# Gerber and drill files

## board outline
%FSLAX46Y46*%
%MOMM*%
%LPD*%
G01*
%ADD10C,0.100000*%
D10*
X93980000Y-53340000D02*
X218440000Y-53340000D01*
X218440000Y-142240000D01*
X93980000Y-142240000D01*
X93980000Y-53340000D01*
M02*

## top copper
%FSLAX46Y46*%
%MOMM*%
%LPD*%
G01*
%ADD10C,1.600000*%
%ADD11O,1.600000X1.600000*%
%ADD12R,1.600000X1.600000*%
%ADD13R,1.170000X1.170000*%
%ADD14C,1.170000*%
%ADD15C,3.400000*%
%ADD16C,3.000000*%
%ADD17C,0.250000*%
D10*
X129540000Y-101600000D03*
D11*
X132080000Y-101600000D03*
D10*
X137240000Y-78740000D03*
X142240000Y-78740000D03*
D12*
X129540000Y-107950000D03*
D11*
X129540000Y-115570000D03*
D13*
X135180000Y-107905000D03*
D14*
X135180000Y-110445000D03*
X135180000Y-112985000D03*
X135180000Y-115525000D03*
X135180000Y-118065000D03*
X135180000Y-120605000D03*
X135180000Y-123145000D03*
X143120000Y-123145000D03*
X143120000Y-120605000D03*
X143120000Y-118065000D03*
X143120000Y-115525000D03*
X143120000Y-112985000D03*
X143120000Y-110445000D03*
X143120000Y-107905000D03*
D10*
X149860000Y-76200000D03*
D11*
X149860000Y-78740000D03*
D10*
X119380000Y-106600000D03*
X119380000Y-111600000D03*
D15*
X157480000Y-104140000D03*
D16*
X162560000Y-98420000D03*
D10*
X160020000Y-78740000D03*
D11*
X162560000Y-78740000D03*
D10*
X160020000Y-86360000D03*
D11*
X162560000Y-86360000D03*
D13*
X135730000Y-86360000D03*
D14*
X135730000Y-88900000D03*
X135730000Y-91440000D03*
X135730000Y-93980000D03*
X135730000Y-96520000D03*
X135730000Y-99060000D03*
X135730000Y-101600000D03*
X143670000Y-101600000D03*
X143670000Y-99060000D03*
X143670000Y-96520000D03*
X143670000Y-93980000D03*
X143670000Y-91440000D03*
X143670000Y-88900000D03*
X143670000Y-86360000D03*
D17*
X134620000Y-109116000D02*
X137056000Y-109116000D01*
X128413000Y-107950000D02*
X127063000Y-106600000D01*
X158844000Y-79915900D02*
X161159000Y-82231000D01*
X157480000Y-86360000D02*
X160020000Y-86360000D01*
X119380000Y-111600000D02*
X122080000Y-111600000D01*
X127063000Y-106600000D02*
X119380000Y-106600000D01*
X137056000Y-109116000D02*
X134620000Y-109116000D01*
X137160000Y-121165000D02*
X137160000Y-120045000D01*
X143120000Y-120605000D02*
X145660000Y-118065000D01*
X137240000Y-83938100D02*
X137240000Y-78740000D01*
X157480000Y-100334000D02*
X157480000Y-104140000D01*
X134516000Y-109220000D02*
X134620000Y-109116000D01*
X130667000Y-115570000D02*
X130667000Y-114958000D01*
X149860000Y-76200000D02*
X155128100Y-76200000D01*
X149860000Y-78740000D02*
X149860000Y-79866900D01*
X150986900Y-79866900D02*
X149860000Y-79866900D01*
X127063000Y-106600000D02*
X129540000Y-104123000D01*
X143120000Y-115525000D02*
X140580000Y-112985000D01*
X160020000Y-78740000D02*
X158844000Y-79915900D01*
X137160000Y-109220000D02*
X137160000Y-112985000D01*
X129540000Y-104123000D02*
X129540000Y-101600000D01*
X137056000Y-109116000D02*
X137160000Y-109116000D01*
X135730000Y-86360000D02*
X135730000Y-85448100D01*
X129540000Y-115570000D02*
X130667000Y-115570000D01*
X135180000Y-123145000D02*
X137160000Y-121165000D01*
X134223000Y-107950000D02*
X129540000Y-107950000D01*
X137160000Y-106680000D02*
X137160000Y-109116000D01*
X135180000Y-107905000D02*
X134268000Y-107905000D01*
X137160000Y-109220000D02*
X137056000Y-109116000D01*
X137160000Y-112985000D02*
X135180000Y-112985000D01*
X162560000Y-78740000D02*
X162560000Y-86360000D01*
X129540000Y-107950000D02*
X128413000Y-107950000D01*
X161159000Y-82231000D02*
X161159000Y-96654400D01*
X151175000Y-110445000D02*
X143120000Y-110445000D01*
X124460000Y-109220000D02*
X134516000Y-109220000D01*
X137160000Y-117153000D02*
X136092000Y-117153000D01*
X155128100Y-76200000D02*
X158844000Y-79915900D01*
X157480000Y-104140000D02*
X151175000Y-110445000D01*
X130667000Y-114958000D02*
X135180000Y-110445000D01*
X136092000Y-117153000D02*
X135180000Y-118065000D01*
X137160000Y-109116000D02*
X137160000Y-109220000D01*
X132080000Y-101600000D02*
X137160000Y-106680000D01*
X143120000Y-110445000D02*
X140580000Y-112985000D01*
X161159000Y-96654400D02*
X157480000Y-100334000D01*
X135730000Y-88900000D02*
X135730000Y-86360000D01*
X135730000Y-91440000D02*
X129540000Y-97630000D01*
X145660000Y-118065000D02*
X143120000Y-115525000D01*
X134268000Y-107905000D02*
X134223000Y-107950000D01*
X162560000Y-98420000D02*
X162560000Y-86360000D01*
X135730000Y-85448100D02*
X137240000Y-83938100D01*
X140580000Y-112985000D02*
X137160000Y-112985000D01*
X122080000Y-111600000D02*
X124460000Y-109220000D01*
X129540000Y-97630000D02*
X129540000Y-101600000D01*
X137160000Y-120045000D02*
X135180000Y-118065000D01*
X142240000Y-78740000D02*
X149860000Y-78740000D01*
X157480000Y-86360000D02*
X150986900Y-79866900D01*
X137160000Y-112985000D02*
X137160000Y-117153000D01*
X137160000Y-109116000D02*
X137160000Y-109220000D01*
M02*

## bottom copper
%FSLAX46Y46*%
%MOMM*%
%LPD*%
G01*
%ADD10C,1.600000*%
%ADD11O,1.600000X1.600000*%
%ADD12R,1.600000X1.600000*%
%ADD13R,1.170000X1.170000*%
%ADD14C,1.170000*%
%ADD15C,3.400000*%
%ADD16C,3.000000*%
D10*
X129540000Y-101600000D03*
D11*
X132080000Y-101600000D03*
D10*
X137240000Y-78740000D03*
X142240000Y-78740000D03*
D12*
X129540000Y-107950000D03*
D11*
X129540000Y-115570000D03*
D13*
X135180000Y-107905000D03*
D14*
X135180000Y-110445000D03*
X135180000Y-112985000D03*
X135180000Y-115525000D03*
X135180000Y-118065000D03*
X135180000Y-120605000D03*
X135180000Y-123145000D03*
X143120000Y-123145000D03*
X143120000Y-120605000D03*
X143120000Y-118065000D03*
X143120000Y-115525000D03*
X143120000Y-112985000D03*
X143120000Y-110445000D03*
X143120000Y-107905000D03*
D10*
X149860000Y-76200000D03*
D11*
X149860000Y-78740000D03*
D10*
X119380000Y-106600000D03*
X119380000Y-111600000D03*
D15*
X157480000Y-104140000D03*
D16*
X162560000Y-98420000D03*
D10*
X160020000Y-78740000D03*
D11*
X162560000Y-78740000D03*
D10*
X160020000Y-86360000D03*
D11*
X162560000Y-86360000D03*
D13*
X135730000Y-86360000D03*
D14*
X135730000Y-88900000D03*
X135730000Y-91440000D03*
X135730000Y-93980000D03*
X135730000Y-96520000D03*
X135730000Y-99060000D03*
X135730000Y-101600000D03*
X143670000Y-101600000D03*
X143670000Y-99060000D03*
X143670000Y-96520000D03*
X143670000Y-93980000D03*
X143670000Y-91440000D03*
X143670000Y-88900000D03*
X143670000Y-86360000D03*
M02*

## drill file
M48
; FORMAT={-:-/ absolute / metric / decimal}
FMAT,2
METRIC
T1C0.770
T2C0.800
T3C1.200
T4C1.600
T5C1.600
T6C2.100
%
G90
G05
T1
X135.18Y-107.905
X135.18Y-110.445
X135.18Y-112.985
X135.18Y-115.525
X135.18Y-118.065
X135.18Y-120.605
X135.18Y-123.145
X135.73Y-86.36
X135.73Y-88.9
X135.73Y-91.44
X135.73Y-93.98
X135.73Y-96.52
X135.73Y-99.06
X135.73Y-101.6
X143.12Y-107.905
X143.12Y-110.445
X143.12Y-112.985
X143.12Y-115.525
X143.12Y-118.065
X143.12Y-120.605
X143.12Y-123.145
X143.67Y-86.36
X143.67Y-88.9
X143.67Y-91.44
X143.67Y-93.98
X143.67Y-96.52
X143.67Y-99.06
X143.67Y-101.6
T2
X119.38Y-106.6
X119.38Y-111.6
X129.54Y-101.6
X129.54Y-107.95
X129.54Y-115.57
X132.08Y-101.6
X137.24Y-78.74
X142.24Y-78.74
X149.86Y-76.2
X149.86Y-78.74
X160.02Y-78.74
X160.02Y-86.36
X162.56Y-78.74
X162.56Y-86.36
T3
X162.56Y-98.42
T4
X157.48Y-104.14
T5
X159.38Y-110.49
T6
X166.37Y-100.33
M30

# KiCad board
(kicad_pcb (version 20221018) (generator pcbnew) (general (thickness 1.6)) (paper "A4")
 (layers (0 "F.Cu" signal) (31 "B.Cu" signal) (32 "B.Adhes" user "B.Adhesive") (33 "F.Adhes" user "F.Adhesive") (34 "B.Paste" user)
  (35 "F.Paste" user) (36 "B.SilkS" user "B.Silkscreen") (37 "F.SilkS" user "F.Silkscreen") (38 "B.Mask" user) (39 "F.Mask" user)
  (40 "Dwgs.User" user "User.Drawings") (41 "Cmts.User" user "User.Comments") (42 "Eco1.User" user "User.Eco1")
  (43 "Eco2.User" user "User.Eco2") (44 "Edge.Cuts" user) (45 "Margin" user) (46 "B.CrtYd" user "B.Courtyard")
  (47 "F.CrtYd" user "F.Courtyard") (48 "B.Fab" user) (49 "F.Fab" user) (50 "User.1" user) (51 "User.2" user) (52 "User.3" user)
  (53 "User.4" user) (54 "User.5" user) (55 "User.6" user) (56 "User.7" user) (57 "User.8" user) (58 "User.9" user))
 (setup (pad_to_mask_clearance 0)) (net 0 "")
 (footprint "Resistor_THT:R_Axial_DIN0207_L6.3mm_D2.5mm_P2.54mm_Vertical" (layer "F.Cu") (at 129.54 101.6)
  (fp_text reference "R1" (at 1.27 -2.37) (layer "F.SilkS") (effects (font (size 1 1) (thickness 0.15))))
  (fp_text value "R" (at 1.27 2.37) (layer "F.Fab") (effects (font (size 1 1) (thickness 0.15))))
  (pad "1" thru_hole circle (at 0 0) (size 1.6 1.6) (drill 0.8) (layers "*.Cu" "*.Mask"))
  (pad "2" thru_hole oval (at 2.54 0) (size 1.6 1.6) (drill 0.8) (layers "*.Cu" "*.Mask")))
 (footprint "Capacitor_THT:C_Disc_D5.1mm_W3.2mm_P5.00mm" (layer "F.Cu") (at 137.24 78.74)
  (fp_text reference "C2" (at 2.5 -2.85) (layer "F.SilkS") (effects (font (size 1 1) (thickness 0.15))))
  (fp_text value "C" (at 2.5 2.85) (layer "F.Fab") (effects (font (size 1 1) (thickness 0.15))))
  (pad "1" thru_hole circle (at 0 0) (size 1.6 1.6) (drill 0.8) (layers "*.Cu" "*.Mask"))
  (pad "2" thru_hole circle (at 5 0) (size 1.6 1.6) (drill 0.8) (layers "*.Cu" "*.Mask")))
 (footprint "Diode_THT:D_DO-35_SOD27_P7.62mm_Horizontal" (layer "F.Cu") (at 129.54 107.95 -90)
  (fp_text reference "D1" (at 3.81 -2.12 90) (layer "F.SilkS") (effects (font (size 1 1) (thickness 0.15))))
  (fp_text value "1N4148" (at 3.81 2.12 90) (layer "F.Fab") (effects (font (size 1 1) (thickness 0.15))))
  (pad "1" thru_hole rect (at 0 0 270) (size 1.6 1.6) (drill 0.8) (layers "*.Cu" "*.Mask"))
  (pad "2" thru_hole oval (at 7.62 0 270) (size 1.6 1.6) (drill 0.8) (layers "*.Cu" "*.Mask")))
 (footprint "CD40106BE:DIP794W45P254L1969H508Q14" (layer "F.Cu") (at 139.15 115.525)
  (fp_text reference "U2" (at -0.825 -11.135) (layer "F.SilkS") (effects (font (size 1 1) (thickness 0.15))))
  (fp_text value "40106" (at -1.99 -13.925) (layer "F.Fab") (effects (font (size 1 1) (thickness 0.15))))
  (pad "1" thru_hole rect (at -3.97 -7.62) (size 1.17 1.17) (drill 0.77) (layers "*.Cu" "*.Mask") (solder_mask_margin 0.102))
  (pad "2" thru_hole circle (at -3.97 -5.08) (size 1.17 1.17) (drill 0.77) (layers "*.Cu" "*.Mask") (solder_mask_margin 0.102))
  (pad "3" thru_hole circle (at -3.97 -2.54) (size 1.17 1.17) (drill 0.77) (layers "*.Cu" "*.Mask") (solder_mask_margin 0.102))
  (pad "4" thru_hole circle (at -3.97 0) (size 1.17 1.17) (drill 0.77) (layers "*.Cu" "*.Mask") (solder_mask_margin 0.102))
  (pad "5" thru_hole circle (at -3.97 2.54) (size 1.17 1.17) (drill 0.77) (layers "*.Cu" "*.Mask") (solder_mask_margin 0.102))
  (pad "6" thru_hole circle (at -3.97 5.08) (size 1.17 1.17) (drill 0.77) (layers "*.Cu" "*.Mask") (solder_mask_margin 0.102))
  (pad "7" thru_hole circle (at -3.97 7.62) (size 1.17 1.17) (drill 0.77) (layers "*.Cu" "*.Mask") (solder_mask_margin 0.102))
  (pad "8" thru_hole circle (at 3.97 7.62) (size 1.17 1.17) (drill 0.77) (layers "*.Cu" "*.Mask") (solder_mask_margin 0.102))
  (pad "9" thru_hole circle (at 3.97 5.08) (size 1.17 1.17) (drill 0.77) (layers "*.Cu" "*.Mask") (solder_mask_margin 0.102))
  (pad "10" thru_hole circle (at 3.97 2.54) (size 1.17 1.17) (drill 0.77) (layers "*.Cu" "*.Mask") (solder_mask_margin 0.102))
  (pad "11" thru_hole circle (at 3.97 0) (size 1.17 1.17) (drill 0.77) (layers "*.Cu" "*.Mask") (solder_mask_margin 0.102))
  (pad "12" thru_hole circle (at 3.97 -2.54) (size 1.17 1.17) (drill 0.77) (layers "*.Cu" "*.Mask") (solder_mask_margin 0.102))
  (pad "13" thru_hole circle (at 3.97 -5.08) (size 1.17 1.17) (drill 0.77) (layers "*.Cu" "*.Mask") (solder_mask_margin 0.102))
  (pad "14" thru_hole circle (at 3.97 -7.62) (size 1.17 1.17) (drill 0.77) (layers "*.Cu" "*.Mask") (solder_mask_margin 0.102)))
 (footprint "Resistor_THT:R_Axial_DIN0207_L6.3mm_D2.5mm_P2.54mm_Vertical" (layer "F.Cu") (at 149.86 76.2 -90)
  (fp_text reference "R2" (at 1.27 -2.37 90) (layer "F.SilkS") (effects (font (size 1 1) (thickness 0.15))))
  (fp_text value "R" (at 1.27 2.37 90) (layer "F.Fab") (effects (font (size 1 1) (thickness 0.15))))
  (pad "1" thru_hole circle (at 0 0 270) (size 1.6 1.6) (drill 0.8) (layers "*.Cu" "*.Mask"))
  (pad "2" thru_hole oval (at 2.54 0 270) (size 1.6 1.6) (drill 0.8) (layers "*.Cu" "*.Mask")))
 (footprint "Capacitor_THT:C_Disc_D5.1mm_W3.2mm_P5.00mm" (layer "F.Cu") (at 119.38 106.6 -90)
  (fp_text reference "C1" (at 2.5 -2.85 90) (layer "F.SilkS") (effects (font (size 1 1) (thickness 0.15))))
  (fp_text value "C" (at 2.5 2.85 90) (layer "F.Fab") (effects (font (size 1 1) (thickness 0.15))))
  (pad "1" thru_hole circle (at 0 0 270) (size 1.6 1.6) (drill 0.8) (layers "*.Cu" "*.Mask"))
  (pad "2" thru_hole circle (at 5 0 270) (size 1.6 1.6) (drill 0.8) (layers "*.Cu" "*.Mask")))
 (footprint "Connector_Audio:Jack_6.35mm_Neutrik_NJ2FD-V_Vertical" (layer "F.Cu") (at 162.56 98.42)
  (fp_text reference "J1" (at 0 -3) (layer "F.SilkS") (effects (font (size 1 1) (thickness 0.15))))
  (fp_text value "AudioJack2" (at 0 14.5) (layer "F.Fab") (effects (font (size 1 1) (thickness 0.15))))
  (pad "" np_thru_hole circle (at -3.18 12.07 180) (size 1.6 1.6) (drill 1.6) (layers "F&B.Cu" "*.Mask"))
  (pad "" np_thru_hole circle (at 3.81 1.91 180) (size 2.1 2.1) (drill 2.1) (layers "F&B.Cu" "*.Mask"))
  (pad "S" thru_hole circle (at -5.08 5.72 180) (size 3.4 3.4) (drill 1.6) (layers "*.Cu" "*.Mask"))
  (pad "T" thru_hole circle (at 0 0 180) (size 3 3) (drill 1.2) (layers "*.Cu" "*.Mask")))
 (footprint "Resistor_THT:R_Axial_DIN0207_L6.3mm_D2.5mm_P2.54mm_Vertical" (layer "F.Cu") (at 160.02 78.74)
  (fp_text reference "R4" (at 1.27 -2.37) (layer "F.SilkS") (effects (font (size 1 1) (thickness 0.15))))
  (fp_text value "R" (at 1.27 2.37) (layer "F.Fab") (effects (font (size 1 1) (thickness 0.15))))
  (pad "1" thru_hole circle (at 0 0) (size 1.6 1.6) (drill 0.8) (layers "*.Cu" "*.Mask"))
  (pad "2" thru_hole oval (at 2.54 0) (size 1.6 1.6) (drill 0.8) (layers "*.Cu" "*.Mask")))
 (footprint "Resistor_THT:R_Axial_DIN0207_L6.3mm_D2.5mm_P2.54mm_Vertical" (layer "F.Cu") (at 160.02 86.36)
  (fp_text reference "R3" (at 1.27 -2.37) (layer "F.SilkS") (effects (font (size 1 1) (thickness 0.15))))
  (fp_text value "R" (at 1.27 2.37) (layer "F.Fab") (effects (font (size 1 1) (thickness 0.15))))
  (pad "1" thru_hole circle (at 0 0) (size 1.6 1.6) (drill 0.8) (layers "*.Cu" "*.Mask"))
  (pad "2" thru_hole oval (at 2.54 0) (size 1.6 1.6) (drill 0.8) (layers "*.Cu" "*.Mask")))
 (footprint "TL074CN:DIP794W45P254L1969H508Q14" (layer "F.Cu") (at 139.7 93.98)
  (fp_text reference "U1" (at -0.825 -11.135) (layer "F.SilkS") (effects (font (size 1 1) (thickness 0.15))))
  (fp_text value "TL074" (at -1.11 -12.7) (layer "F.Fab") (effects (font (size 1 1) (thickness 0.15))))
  (pad "1" thru_hole rect (at -3.97 -7.62) (size 1.17 1.17) (drill 0.77) (layers "*.Cu" "*.Mask") (solder_mask_margin 0.102))
  (pad "2" thru_hole circle (at -3.97 -5.08) (size 1.17 1.17) (drill 0.77) (layers "*.Cu" "*.Mask") (solder_mask_margin 0.102))
  (pad "3" thru_hole circle (at -3.97 -2.54) (size 1.17 1.17) (drill 0.77) (layers "*.Cu" "*.Mask") (solder_mask_margin 0.102))
  (pad "4" thru_hole circle (at -3.97 0) (size 1.17 1.17) (drill 0.77) (layers "*.Cu" "*.Mask") (solder_mask_margin 0.102))
  (pad "5" thru_hole circle (at -3.97 2.54) (size 1.17 1.17) (drill 0.77) (layers "*.Cu" "*.Mask") (solder_mask_margin 0.102))
  (pad "6" thru_hole circle (at -3.97 5.08) (size 1.17 1.17) (drill 0.77) (layers "*.Cu" "*.Mask") (solder_mask_margin 0.102))
  (pad "7" thru_hole circle (at -3.97 7.62) (size 1.17 1.17) (drill 0.77) (layers "*.Cu" "*.Mask") (solder_mask_margin 0.102))
  (pad "8" thru_hole circle (at 3.97 7.62) (size 1.17 1.17) (drill 0.77) (layers "*.Cu" "*.Mask") (solder_mask_margin 0.102))
  (pad "9" thru_hole circle (at 3.97 5.08) (size 1.17 1.17) (drill 0.77) (layers "*.Cu" "*.Mask") (solder_mask_margin 0.102))
  (pad "10" thru_hole circle (at 3.97 2.54) (size 1.17 1.17) (drill 0.77) (layers "*.Cu" "*.Mask") (solder_mask_margin 0.102))
  (pad "11" thru_hole circle (at 3.97 0) (size 1.17 1.17) (drill 0.77) (layers "*.Cu" "*.Mask") (solder_mask_margin 0.102))
  (pad "12" thru_hole circle (at 3.97 -2.54) (size 1.17 1.17) (drill 0.77) (layers "*.Cu" "*.Mask") (solder_mask_margin 0.102))
  (pad "13" thru_hole circle (at 3.97 -5.08) (size 1.17 1.17) (drill 0.77) (layers "*.Cu" "*.Mask") (solder_mask_margin 0.102))
  (pad "14" thru_hole circle (at 3.97 -7.62) (size 1.17 1.17) (drill 0.77) (layers "*.Cu" "*.Mask") (solder_mask_margin 0.102)))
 (gr_rect (start 93.98 53.34) (end 218.44 142.24) (stroke (width 0.1) (type default)) (fill none) (layer "Edge.Cuts"))
 (segment (start 134.62 109.116) (end 137.056 109.116) (width 0.25) (layer "F.Cu") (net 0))
 (segment (start 128.413 107.95) (end 127.063 106.6) (width 0.25) (layer "F.Cu") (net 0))
 (segment (start 158.844 79.9159) (end 161.159 82.231) (width 0.25) (layer "F.Cu") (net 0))
 (segment (start 157.48 86.36) (end 160.02 86.36) (width 0.25) (layer "F.Cu") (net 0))
 (segment (start 119.38 111.6) (end 122.08 111.6) (width 0.25) (layer "F.Cu") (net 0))
 (segment (start 127.063 106.6) (end 119.38 106.6) (width 0.25) (layer "F.Cu") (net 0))
 (segment (start 137.056 109.116) (end 134.62 109.116) (width 0.25) (layer "F.Cu") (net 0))
 (segment (start 137.16 121.165) (end 137.16 120.045) (width 0.25) (layer "F.Cu") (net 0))
 (segment (start 143.12 120.605) (end 145.66 118.065) (width 0.25) (layer "F.Cu") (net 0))
 (segment (start 137.24 83.9381) (end 137.24 78.74) (width 0.25) (layer "F.Cu") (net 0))
 (segment (start 157.48 100.334) (end 157.48 104.14) (width 0.25) (layer "F.Cu") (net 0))
 (segment (start 134.516 109.22) (end 134.62 109.116) (width 0.25) (layer "F.Cu") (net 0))
 (segment (start 130.667 115.57) (end 130.667 114.958) (width 0.25) (layer "F.Cu") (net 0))
 (segment (start 149.86 76.2) (end 155.1281 76.2) (width 0.25) (layer "F.Cu") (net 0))
 (segment (start 149.86 78.74) (end 149.86 79.8669) (width 0.25) (layer "F.Cu") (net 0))
 (segment (start 150.9869 79.8669) (end 149.86 79.8669) (width 0.25) (layer "F.Cu") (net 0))
 (segment (start 127.063 106.6) (end 129.54 104.123) (width 0.25) (layer "F.Cu") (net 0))
 (segment (start 143.12 115.525) (end 140.58 112.985) (width 0.25) (layer "F.Cu") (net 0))
 (segment (start 160.02 78.74) (end 158.844 79.9159) (width 0.25) (layer "F.Cu") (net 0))
 (segment (start 137.16 109.22) (end 137.16 112.985) (width 0.25) (layer "F.Cu") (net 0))
 (segment (start 129.54 104.123) (end 129.54 101.6) (width 0.25) (layer "F.Cu") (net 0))
 (segment (start 137.056 109.116) (end 137.16 109.116) (width 0.25) (layer "F.Cu") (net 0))
 (segment (start 135.73 86.36) (end 135.73 85.4481) (width 0.25) (layer "F.Cu") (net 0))
 (segment (start 129.54 115.57) (end 130.667 115.57) (width 0.25) (layer "F.Cu") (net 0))
 (segment (start 135.18 123.145) (end 137.16 121.165) (width 0.25) (layer "F.Cu") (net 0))
 (segment (start 134.223 107.95) (end 129.54 107.95) (width 0.25) (layer "F.Cu") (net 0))
 (segment (start 137.16 106.68) (end 137.16 109.116) (width 0.25) (layer "F.Cu") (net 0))
 (segment (start 135.18 107.905) (end 134.268 107.905) (width 0.25) (layer "F.Cu") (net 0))
 (segment (start 137.16 109.22) (end 137.056 109.116) (width 0.25) (layer "F.Cu") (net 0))
 (segment (start 137.16 112.985) (end 135.18 112.985) (width 0.25) (layer "F.Cu") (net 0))
 (segment (start 162.56 78.74) (end 162.56 86.36) (width 0.25) (layer "F.Cu") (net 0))
 (segment (start 129.54 107.95) (end 128.413 107.95) (width 0.25) (layer "F.Cu") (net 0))
 (segment (start 161.159 82.231) (end 161.159 96.6544) (width 0.25) (layer "F.Cu") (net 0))
 (segment (start 151.175 110.445) (end 143.12 110.445) (width 0.25) (layer "F.Cu") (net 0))
 (segment (start 124.46 109.22) (end 134.516 109.22) (width 0.25) (layer "F.Cu") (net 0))
 (segment (start 137.16 117.153) (end 136.092 117.153) (width 0.25) (layer "F.Cu") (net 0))
 (segment (start 155.1281 76.2) (end 158.844 79.9159) (width 0.25) (layer "F.Cu") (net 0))
 (segment (start 157.48 104.14) (end 151.175 110.445) (width 0.25) (layer "F.Cu") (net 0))
 (segment (start 130.667 114.958) (end 135.18 110.445) (width 0.25) (layer "F.Cu") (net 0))
 (segment (start 136.092 117.153) (end 135.18 118.065) (width 0.25) (layer "F.Cu") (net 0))
 (segment (start 137.16 109.116) (end 137.16 109.22) (width 0.25) (layer "F.Cu") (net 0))
 (segment (start 132.08 101.6) (end 137.16 106.68) (width 0.25) (layer "F.Cu") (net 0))
 (segment (start 143.12 110.445) (end 140.58 112.985) (width 0.25) (layer "F.Cu") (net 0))
 (segment (start 161.159 96.6544) (end 157.48 100.334) (width 0.25) (layer "F.Cu") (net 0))
 (segment (start 135.73 88.9) (end 135.73 86.36) (width 0.25) (layer "F.Cu") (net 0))
 (segment (start 135.73 91.44) (end 129.54 97.63) (width 0.25) (layer "F.Cu") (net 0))
 (segment (start 145.66 118.065) (end 143.12 115.525) (width 0.25) (layer "F.Cu") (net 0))
 (segment (start 134.268 107.905) (end 134.223 107.95) (width 0.25) (layer "F.Cu") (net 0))
 (segment (start 162.56 98.42) (end 162.56 86.36) (width 0.25) (layer "F.Cu") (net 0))
 (segment (start 135.73 85.4481) (end 137.24 83.9381) (width 0.25) (layer "F.Cu") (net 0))
 (segment (start 140.58 112.985) (end 137.16 112.985) (width 0.25) (layer "F.Cu") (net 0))
 (segment (start 122.08 111.6) (end 124.46 109.22) (width 0.25) (layer "F.Cu") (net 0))
 (segment (start 129.54 97.63) (end 129.54 101.6) (width 0.25) (layer "F.Cu") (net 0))
 (segment (start 137.16 120.045) (end 135.18 118.065) (width 0.25) (layer "F.Cu") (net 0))
 (segment (start 142.24 78.74) (end 149.86 78.74) (width 0.25) (layer "F.Cu") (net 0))
 (segment (start 157.48 86.36) (end 150.9869 79.8669) (width 0.25) (layer "F.Cu") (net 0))
 (segment (start 137.16 112.985) (end 137.16 117.153) (width 0.25) (layer "F.Cu") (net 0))
 (segment (start 137.16 109.116) (end 137.16 109.22) (width 0.25) (layer "F.Cu") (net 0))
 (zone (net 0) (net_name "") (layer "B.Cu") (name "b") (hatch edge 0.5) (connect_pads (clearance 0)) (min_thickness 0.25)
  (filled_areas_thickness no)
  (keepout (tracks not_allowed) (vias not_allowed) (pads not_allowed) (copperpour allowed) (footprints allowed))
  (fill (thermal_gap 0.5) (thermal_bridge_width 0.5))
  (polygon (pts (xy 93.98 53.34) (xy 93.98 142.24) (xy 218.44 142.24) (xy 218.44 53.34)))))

